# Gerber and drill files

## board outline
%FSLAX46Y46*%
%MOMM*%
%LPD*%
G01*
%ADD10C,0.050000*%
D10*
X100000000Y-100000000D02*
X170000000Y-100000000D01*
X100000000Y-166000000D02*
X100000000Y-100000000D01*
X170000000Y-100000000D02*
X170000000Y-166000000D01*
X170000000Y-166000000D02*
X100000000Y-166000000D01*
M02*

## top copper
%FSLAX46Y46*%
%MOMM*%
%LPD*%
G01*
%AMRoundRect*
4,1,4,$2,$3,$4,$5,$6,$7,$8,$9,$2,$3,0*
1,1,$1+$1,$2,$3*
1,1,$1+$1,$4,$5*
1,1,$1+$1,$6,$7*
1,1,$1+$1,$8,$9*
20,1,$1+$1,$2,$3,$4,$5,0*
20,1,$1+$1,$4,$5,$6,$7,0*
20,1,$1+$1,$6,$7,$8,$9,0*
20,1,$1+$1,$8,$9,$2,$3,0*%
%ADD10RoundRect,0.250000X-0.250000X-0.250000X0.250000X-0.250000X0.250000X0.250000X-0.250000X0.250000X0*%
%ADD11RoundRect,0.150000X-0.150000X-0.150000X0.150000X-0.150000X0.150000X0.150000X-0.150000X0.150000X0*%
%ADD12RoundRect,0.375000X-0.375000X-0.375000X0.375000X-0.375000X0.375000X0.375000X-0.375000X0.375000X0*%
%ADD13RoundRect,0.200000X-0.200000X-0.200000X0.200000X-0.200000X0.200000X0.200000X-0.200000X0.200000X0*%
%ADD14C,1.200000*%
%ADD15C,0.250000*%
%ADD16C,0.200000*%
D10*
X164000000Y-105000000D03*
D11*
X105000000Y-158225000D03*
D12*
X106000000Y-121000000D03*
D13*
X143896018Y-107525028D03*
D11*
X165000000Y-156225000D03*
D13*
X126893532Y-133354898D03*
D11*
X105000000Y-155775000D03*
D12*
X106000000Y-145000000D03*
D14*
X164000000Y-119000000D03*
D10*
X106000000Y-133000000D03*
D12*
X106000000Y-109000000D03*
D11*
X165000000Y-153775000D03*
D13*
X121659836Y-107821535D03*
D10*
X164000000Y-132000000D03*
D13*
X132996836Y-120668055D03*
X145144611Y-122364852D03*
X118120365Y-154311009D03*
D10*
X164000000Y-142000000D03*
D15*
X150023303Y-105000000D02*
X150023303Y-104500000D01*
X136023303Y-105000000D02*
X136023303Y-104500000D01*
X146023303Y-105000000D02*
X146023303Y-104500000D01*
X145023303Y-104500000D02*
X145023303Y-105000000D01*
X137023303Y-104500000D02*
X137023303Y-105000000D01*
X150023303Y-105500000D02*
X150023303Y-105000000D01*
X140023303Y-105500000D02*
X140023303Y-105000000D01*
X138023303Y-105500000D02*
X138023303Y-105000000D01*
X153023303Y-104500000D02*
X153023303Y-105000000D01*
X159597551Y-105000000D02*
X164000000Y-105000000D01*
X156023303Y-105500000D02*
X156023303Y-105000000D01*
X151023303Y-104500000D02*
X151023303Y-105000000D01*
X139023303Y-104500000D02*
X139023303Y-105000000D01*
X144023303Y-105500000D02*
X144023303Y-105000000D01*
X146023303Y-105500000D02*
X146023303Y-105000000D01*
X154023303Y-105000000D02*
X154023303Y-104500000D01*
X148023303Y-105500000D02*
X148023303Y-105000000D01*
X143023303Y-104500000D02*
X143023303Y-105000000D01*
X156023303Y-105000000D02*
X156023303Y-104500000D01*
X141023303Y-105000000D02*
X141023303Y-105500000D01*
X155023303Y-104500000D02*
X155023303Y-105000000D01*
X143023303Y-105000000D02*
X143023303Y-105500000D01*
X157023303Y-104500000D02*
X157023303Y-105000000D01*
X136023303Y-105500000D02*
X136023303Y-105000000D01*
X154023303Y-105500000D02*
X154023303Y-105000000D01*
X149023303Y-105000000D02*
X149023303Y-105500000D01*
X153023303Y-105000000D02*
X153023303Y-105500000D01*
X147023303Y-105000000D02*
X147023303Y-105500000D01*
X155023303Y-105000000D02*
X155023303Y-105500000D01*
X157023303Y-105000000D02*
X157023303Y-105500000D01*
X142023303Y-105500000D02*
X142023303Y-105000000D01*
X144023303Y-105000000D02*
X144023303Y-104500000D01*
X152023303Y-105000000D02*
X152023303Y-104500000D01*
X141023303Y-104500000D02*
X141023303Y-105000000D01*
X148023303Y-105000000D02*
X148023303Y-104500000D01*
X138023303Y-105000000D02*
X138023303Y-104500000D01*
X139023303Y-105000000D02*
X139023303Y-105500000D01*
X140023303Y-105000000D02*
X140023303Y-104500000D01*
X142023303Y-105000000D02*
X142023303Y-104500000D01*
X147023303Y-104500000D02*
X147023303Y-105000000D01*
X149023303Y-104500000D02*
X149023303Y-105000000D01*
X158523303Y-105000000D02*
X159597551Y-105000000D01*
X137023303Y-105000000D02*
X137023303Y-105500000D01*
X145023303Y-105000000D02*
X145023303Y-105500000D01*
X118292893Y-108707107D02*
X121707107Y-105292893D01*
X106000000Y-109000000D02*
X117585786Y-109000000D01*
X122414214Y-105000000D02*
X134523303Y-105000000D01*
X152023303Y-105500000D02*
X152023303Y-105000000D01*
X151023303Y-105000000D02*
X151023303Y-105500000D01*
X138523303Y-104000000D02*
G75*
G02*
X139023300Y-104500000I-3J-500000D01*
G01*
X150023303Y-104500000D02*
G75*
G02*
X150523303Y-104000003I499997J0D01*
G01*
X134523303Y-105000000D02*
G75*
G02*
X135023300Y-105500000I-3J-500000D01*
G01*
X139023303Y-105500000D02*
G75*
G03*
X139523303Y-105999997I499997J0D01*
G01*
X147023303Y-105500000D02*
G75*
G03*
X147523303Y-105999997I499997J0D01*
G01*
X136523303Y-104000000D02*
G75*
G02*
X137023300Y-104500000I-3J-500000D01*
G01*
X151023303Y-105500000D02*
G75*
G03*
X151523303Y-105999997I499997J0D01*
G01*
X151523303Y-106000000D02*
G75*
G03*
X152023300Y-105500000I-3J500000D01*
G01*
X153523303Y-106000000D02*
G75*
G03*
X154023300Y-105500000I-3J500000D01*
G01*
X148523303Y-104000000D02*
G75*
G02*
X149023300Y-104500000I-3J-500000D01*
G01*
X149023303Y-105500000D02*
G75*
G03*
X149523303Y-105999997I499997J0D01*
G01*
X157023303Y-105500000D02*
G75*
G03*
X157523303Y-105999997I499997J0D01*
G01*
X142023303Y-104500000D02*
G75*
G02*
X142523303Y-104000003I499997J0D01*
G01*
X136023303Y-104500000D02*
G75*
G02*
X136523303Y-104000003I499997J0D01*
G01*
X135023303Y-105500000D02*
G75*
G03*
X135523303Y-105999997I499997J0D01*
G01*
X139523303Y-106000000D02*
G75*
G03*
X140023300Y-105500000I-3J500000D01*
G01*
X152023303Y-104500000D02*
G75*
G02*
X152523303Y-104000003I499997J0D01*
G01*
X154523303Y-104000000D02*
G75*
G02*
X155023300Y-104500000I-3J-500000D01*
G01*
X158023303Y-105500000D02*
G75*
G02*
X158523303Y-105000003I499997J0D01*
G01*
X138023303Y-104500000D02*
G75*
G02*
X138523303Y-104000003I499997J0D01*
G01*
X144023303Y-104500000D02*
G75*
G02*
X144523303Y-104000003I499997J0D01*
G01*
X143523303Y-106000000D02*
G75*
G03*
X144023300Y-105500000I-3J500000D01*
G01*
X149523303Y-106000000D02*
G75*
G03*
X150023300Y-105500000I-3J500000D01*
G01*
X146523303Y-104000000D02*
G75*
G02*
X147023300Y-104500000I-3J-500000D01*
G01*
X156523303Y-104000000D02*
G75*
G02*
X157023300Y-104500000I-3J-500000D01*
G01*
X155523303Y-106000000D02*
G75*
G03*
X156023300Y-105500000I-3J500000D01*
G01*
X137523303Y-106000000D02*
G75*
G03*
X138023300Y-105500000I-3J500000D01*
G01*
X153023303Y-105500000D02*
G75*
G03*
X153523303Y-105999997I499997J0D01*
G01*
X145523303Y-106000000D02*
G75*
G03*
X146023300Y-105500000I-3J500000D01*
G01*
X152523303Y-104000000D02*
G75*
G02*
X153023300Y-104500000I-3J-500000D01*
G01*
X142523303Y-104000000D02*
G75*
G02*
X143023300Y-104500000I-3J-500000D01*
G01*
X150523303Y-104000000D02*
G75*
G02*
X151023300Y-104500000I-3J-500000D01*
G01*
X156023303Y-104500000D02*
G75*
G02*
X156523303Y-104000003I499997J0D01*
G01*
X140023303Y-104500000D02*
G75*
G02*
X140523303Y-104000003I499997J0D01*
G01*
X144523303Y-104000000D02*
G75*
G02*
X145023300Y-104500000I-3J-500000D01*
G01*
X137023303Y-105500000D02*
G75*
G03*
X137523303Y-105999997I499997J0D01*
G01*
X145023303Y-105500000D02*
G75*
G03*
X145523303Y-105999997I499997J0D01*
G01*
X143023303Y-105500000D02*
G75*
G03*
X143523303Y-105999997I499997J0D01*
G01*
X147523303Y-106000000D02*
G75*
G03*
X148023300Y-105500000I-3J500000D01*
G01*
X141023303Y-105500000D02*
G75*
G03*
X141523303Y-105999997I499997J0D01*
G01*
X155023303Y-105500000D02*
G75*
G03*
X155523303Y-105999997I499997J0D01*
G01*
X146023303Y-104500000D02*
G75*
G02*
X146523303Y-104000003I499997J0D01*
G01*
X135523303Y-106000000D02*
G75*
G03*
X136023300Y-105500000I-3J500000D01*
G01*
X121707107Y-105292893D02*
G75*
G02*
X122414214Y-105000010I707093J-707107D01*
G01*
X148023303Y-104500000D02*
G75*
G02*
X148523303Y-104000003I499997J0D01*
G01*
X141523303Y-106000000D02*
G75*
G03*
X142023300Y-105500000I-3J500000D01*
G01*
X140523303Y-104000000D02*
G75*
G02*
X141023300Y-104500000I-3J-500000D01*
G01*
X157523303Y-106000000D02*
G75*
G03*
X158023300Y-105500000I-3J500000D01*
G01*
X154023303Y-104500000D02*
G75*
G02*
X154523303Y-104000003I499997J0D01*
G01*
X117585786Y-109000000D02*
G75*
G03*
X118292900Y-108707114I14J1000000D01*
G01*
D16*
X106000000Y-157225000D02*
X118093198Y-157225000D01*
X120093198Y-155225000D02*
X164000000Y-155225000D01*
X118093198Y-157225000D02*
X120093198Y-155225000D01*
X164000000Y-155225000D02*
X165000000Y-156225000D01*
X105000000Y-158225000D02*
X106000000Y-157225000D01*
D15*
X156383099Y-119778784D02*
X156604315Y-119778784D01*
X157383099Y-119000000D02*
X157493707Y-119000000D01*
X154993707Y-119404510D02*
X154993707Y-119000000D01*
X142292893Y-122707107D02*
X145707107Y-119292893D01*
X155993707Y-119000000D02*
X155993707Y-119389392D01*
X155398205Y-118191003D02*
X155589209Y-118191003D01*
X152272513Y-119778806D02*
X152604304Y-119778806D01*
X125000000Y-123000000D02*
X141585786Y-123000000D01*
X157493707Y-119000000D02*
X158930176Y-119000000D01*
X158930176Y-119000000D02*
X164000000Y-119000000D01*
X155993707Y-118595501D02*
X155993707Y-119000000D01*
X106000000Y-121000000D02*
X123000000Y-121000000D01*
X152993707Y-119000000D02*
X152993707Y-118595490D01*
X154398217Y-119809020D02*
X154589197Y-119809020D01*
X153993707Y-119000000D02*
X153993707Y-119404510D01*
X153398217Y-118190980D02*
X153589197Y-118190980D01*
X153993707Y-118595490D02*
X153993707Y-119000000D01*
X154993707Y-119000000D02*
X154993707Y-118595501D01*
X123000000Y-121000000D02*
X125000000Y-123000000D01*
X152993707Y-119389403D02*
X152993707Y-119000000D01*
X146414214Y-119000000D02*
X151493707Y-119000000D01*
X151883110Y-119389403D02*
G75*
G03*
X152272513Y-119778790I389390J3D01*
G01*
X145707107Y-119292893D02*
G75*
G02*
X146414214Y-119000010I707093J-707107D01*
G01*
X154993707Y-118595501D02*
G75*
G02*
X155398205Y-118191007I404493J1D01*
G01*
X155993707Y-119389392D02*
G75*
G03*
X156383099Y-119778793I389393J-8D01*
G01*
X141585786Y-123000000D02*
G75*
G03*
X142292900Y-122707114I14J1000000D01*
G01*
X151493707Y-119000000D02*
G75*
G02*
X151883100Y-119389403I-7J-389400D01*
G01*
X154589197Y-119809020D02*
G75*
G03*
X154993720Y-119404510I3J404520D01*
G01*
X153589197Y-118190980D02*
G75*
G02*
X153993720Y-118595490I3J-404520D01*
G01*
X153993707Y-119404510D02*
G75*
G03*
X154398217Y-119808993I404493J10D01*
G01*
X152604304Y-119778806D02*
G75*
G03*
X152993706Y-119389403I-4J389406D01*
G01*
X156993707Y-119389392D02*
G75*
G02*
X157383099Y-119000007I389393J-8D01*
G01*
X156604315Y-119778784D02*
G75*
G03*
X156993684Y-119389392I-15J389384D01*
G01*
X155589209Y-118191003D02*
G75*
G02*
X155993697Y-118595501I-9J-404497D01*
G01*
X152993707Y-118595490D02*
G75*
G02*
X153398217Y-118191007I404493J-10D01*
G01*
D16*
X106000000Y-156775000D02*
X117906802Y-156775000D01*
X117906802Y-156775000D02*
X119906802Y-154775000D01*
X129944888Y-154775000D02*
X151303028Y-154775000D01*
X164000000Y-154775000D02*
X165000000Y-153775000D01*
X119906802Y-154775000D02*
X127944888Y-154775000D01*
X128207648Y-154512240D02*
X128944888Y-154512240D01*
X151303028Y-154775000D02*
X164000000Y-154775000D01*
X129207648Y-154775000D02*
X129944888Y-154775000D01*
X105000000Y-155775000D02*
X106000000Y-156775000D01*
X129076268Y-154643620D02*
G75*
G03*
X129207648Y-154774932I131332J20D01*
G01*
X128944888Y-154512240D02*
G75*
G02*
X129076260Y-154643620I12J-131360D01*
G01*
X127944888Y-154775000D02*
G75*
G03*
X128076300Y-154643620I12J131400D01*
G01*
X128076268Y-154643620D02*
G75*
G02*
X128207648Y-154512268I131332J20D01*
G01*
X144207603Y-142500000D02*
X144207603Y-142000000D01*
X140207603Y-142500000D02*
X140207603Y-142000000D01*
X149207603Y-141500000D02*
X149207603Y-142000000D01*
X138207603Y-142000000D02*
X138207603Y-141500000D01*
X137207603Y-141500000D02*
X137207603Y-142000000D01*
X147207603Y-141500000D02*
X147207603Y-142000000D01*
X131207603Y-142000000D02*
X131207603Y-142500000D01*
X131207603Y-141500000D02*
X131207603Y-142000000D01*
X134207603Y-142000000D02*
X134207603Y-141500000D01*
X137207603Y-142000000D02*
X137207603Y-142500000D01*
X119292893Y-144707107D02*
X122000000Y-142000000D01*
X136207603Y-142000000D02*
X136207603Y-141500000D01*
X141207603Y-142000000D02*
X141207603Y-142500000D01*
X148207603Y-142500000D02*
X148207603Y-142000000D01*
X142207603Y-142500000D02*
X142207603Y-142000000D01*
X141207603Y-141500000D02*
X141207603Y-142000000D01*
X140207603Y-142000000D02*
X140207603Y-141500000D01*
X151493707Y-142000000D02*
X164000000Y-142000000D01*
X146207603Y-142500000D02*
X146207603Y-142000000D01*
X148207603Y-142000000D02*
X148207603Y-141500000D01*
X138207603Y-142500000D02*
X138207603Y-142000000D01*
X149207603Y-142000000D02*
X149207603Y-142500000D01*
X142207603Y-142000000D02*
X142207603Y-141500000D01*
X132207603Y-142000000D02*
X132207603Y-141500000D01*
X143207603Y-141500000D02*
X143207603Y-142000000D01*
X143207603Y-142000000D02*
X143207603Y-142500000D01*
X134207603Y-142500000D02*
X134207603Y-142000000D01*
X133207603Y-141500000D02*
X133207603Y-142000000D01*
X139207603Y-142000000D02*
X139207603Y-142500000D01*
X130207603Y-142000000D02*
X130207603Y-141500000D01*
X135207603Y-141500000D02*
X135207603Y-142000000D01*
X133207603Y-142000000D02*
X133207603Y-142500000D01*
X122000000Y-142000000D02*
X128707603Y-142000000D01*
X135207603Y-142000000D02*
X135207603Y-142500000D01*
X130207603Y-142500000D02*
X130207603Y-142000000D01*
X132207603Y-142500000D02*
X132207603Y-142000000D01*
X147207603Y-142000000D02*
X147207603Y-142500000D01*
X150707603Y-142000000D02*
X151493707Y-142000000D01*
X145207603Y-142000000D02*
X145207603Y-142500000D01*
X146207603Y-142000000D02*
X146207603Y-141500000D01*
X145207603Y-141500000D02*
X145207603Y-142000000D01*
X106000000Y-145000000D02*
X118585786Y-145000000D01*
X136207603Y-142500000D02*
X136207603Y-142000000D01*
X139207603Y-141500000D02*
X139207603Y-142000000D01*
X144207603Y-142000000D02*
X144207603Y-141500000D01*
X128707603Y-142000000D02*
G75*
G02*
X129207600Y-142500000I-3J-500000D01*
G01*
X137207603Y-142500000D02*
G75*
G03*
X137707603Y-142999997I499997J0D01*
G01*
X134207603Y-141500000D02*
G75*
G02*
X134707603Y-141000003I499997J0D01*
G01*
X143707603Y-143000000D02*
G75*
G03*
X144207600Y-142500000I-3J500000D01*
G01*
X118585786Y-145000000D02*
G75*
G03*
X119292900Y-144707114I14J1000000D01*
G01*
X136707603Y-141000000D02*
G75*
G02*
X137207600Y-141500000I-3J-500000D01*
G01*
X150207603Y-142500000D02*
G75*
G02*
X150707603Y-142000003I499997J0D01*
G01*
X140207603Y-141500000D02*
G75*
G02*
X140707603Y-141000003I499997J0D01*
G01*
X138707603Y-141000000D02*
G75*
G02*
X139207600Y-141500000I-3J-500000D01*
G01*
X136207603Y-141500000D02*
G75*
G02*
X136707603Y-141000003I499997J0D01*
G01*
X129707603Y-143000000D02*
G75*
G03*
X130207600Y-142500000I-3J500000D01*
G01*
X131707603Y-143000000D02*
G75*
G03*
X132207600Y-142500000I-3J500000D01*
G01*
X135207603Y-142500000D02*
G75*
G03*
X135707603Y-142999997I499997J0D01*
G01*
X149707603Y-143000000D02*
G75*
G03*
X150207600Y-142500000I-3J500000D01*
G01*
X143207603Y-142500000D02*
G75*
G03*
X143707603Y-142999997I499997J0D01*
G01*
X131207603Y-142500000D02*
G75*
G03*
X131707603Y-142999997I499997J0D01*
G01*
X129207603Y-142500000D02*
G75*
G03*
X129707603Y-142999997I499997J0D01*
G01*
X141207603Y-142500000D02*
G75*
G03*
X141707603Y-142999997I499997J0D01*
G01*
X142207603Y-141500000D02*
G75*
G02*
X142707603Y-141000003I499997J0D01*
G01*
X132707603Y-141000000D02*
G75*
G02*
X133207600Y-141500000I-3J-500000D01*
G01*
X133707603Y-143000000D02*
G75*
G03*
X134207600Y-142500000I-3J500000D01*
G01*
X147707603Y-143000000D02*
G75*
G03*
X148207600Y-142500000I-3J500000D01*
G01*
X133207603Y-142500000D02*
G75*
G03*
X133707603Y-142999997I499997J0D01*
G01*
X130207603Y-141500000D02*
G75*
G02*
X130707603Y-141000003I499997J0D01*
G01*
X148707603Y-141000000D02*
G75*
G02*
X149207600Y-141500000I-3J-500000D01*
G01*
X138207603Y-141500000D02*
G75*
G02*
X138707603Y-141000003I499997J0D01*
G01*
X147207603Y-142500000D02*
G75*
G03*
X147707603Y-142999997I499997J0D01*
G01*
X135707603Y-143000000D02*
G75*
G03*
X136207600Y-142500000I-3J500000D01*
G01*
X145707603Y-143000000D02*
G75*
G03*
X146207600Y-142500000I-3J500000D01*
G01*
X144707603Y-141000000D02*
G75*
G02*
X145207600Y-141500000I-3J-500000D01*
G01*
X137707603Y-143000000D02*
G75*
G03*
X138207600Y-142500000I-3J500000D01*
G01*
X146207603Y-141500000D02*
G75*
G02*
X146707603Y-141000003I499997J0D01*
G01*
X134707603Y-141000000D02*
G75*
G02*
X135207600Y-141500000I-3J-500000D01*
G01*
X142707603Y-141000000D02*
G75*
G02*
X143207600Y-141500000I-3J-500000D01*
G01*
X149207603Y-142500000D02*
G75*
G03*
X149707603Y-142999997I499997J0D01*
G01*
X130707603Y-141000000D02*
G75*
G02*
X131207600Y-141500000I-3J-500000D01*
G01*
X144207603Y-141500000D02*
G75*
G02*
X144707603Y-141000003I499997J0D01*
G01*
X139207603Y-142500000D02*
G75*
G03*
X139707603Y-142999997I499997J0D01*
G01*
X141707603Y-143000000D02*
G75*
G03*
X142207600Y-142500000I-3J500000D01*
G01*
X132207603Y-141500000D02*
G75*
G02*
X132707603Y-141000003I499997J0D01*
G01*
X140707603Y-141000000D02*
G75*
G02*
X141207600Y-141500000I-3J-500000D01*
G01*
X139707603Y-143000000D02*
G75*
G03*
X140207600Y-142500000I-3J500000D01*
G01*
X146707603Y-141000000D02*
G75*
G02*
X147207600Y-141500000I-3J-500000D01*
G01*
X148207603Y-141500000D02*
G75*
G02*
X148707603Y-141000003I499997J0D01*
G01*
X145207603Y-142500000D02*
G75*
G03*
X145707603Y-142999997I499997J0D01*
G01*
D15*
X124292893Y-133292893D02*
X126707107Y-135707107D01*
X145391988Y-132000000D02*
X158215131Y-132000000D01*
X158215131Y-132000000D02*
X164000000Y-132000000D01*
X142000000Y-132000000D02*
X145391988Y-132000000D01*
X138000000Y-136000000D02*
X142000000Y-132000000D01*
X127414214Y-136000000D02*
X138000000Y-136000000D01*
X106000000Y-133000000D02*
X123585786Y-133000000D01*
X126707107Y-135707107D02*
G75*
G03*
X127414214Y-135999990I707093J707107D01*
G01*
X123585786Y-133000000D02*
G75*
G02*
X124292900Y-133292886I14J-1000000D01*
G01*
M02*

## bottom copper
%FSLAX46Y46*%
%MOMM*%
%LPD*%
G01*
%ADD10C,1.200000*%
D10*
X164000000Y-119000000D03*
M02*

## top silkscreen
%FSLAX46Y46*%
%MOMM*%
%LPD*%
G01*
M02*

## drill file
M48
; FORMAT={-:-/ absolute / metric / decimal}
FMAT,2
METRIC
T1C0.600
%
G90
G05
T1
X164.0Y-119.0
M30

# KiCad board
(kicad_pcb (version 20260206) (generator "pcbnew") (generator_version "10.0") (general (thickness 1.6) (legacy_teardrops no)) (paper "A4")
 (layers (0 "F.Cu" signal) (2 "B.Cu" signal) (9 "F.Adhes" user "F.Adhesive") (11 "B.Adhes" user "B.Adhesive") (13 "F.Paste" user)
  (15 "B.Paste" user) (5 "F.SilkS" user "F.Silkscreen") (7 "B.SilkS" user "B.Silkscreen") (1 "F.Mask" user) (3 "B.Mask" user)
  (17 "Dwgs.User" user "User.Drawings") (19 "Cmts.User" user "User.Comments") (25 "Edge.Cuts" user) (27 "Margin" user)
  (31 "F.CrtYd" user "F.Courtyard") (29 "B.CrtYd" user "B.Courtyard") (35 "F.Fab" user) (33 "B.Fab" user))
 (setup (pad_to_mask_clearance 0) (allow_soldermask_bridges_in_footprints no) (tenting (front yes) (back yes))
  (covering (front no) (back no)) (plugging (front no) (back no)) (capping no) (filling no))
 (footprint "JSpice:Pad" (layer "F.Cu") (at 164 105)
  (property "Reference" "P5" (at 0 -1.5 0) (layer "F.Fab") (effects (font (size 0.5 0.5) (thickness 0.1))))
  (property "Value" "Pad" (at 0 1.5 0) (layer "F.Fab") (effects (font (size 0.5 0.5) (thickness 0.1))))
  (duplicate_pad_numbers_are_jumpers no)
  (pad "1" smd roundrect (at 0 0) (size 1 1) (layers "F.Cu" "F.Mask") (roundrect_rratio 0.25) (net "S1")))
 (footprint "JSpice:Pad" (layer "F.Cu") (at 105 158.225)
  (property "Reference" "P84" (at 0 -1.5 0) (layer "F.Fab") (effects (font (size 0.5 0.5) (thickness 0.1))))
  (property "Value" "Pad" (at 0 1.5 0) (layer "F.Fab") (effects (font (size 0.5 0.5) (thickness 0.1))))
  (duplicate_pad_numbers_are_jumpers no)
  (pad "1" smd roundrect (at 0 0) (size 0.6 0.6) (layers "F.Cu" "F.Mask") (roundrect_rratio 0.25) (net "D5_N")))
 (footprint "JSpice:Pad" (layer "F.Cu") (at 106 121)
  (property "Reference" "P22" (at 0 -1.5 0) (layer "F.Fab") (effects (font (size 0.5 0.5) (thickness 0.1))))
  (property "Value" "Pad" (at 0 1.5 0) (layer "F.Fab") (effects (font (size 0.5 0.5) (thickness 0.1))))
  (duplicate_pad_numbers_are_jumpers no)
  (pad "1" smd roundrect (at 0 0) (size 1.5 1.5) (layers "F.Cu" "F.Mask") (roundrect_rratio 0.25) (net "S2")))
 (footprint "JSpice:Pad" (layer "F.Cu") (at 143.896018 107.525028)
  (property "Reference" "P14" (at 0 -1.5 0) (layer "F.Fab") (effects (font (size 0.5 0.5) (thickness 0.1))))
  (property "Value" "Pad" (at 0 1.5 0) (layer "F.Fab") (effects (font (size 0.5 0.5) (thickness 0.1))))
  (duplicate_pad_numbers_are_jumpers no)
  (pad "1" smd roundrect (at 0 0) (size 0.8 0.8) (layers "F.Cu" "F.Mask") (roundrect_rratio 0.25) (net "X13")))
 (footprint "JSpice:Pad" (layer "F.Cu") (at 165 156.225)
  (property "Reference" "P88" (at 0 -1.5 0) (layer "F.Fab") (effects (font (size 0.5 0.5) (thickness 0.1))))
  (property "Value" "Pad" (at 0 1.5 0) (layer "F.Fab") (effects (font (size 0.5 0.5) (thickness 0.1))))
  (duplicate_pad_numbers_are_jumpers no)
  (pad "1" smd roundrect (at 0 0) (size 0.6 0.6) (layers "F.Cu" "F.Mask") (roundrect_rratio 0.25) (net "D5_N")))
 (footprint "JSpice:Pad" (layer "F.Cu") (at 126.893532 133.354898)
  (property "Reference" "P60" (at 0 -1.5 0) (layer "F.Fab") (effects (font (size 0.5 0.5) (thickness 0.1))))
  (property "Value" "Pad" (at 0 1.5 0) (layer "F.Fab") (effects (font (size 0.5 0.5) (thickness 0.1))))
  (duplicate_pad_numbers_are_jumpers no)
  (pad "1" smd roundrect (at 0 0) (size 0.8 0.8) (layers "F.Cu" "F.Mask") (roundrect_rratio 0.25) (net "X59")))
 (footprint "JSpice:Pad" (layer "F.Cu") (at 105 155.775)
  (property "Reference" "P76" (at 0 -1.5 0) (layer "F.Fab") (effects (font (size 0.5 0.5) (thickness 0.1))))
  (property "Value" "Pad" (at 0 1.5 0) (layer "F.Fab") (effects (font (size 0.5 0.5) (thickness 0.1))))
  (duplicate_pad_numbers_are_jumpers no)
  (pad "1" smd roundrect (at 0 0) (size 0.6 0.6) (layers "F.Cu" "F.Mask") (roundrect_rratio 0.25) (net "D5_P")))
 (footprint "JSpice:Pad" (layer "F.Cu") (at 106 145)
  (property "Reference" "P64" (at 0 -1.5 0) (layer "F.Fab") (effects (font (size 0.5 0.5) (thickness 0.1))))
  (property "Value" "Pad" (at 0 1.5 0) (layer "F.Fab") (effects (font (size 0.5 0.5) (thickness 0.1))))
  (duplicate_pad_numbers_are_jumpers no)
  (pad "1" smd roundrect (at 0 0) (size 1.5 1.5) (layers "F.Cu" "F.Mask") (roundrect_rratio 0.25) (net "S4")))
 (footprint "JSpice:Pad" (layer "F.Cu") (at 164 119)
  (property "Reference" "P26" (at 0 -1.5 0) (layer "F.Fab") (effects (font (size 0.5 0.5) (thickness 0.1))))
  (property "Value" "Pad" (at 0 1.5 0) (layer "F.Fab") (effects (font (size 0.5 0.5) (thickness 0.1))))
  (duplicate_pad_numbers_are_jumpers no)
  (pad "1" thru_hole circle (at 0 0) (size 1.2 1.2) (drill 0.6) (layers "*.Cu" "*.Mask") (remove_unused_layers no) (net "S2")))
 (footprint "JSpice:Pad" (layer "F.Cu") (at 106 133)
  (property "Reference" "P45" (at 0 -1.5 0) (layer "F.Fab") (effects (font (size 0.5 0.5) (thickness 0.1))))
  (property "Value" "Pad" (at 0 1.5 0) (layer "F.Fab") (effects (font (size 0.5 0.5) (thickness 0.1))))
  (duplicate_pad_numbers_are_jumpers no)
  (pad "1" smd roundrect (at 0 0) (size 1 1) (layers "F.Cu" "F.Mask") (roundrect_rratio 0.25) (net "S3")))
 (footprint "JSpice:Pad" (layer "F.Cu") (at 106 109)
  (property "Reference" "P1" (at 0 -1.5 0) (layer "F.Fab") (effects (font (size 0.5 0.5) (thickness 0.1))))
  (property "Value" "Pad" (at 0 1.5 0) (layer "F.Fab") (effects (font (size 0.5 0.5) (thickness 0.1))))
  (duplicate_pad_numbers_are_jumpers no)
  (pad "1" smd roundrect (at 0 0) (size 1.5 1.5) (layers "F.Cu" "F.Mask") (roundrect_rratio 0.25) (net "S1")))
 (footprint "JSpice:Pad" (layer "F.Cu") (at 165 153.775)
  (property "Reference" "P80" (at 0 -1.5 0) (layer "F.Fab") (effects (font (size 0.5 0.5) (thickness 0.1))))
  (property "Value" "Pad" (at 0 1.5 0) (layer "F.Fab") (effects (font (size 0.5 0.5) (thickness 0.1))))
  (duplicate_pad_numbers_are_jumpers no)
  (pad "1" smd roundrect (at 0 0) (size 0.6 0.6) (layers "F.Cu" "F.Mask") (roundrect_rratio 0.25) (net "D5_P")))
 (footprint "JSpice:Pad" (layer "F.Cu") (at 121.659836 107.821535)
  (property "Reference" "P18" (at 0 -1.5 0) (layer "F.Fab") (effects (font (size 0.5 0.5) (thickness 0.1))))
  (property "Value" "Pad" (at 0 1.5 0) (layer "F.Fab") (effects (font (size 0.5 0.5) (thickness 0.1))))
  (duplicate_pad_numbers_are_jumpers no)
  (pad "1" smd roundrect (at 0 0) (size 0.8 0.8) (layers "F.Cu" "F.Mask") (roundrect_rratio 0.25) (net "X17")))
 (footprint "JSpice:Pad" (layer "F.Cu") (at 164 132)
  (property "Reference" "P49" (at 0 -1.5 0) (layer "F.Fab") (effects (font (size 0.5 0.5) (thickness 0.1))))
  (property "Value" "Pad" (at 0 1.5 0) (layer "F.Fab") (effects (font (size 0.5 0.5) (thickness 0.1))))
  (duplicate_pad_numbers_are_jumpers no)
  (pad "1" smd roundrect (at 0 0) (size 1 1) (layers "F.Cu" "F.Mask") (roundrect_rratio 0.25) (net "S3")))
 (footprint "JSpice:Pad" (layer "F.Cu") (at 132.996836 120.668055)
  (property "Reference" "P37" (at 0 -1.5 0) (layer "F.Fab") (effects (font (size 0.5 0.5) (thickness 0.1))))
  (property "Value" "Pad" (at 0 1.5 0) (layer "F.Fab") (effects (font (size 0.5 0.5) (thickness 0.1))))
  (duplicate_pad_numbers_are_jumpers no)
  (pad "1" smd roundrect (at 0 0) (size 0.8 0.8) (layers "F.Cu" "F.Mask") (roundrect_rratio 0.25) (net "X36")))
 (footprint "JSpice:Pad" (layer "F.Cu") (at 145.144611 122.364852)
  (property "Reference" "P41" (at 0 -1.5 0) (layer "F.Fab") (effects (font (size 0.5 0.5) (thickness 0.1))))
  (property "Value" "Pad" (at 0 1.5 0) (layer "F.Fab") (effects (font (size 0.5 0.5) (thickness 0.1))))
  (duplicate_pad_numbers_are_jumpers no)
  (pad "1" smd roundrect (at 0 0) (size 0.8 0.8) (layers "F.Cu" "F.Mask") (roundrect_rratio 0.25) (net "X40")))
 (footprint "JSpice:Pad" (layer "F.Cu") (at 118.120365 154.311009)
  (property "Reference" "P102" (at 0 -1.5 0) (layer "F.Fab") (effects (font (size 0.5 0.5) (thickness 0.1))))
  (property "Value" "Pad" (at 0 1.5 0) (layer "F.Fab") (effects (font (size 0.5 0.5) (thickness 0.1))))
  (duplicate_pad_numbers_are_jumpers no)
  (pad "1" smd roundrect (at 0 0) (size 0.8 0.8) (layers "F.Cu" "F.Mask") (roundrect_rratio 0.25) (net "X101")))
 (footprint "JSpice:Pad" (layer "F.Cu") (at 164 142)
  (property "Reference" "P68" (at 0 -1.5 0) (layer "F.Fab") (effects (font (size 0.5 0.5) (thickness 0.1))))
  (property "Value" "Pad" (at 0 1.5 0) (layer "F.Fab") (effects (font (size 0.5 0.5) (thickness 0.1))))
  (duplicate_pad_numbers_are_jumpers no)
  (pad "1" smd roundrect (at 0 0) (size 1 1) (layers "F.Cu" "F.Mask") (roundrect_rratio 0.25) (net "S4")))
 (gr_line (start 100 100) (end 170 100) (stroke (width 0.05) (type default)) (layer "Edge.Cuts"))
 (gr_line (start 100 166) (end 100 100) (stroke (width 0.05) (type default)) (layer "Edge.Cuts"))
 (gr_line (start 170 100) (end 170 166) (stroke (width 0.05) (type default)) (layer "Edge.Cuts"))
 (gr_line (start 170 166) (end 100 166) (stroke (width 0.05) (type default)) (layer "Edge.Cuts"))
 (segment (start 150.023303 105) (end 150.023303 104.5) (width 0.25) (layer "F.Cu") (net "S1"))
 (segment (start 136.023303 105) (end 136.023303 104.5) (width 0.25) (layer "F.Cu") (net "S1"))
 (segment (start 146.023303 105) (end 146.023303 104.5) (width 0.25) (layer "F.Cu") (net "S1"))
 (segment (start 145.023303 104.5) (end 145.023303 105) (width 0.25) (layer "F.Cu") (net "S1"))
 (segment (start 137.023303 104.5) (end 137.023303 105) (width 0.25) (layer "F.Cu") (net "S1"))
 (segment (start 150.023303 105.5) (end 150.023303 105) (width 0.25) (layer "F.Cu") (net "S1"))
 (segment (start 140.023303 105.5) (end 140.023303 105) (width 0.25) (layer "F.Cu") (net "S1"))
 (segment (start 138.023303 105.5) (end 138.023303 105) (width 0.25) (layer "F.Cu") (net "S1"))
 (segment (start 153.023303 104.5) (end 153.023303 105) (width 0.25) (layer "F.Cu") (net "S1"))
 (segment (start 159.597551 105) (end 164 105) (width 0.25) (layer "F.Cu") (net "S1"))
 (segment (start 156.023303 105.5) (end 156.023303 105) (width 0.25) (layer "F.Cu") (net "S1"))
 (segment (start 151.023303 104.5) (end 151.023303 105) (width 0.25) (layer "F.Cu") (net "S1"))
 (segment (start 139.023303 104.5) (end 139.023303 105) (width 0.25) (layer "F.Cu") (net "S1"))
 (segment (start 144.023303 105.5) (end 144.023303 105) (width 0.25) (layer "F.Cu") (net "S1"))
 (segment (start 146.023303 105.5) (end 146.023303 105) (width 0.25) (layer "F.Cu") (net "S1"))
 (segment (start 154.023303 105) (end 154.023303 104.5) (width 0.25) (layer "F.Cu") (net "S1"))
 (segment (start 148.023303 105.5) (end 148.023303 105) (width 0.25) (layer "F.Cu") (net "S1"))
 (segment (start 143.023303 104.5) (end 143.023303 105) (width 0.25) (layer "F.Cu") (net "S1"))
 (segment (start 156.023303 105) (end 156.023303 104.5) (width 0.25) (layer "F.Cu") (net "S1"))
 (segment (start 141.023303 105) (end 141.023303 105.5) (width 0.25) (layer "F.Cu") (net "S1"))
 (segment (start 155.023303 104.5) (end 155.023303 105) (width 0.25) (layer "F.Cu") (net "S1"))
 (segment (start 143.023303 105) (end 143.023303 105.5) (width 0.25) (layer "F.Cu") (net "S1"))
 (segment (start 157.023303 104.5) (end 157.023303 105) (width 0.25) (layer "F.Cu") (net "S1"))
 (segment (start 136.023303 105.5) (end 136.023303 105) (width 0.25) (layer "F.Cu") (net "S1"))
 (segment (start 154.023303 105.5) (end 154.023303 105) (width 0.25) (layer "F.Cu") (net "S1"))
 (segment (start 149.023303 105) (end 149.023303 105.5) (width 0.25) (layer "F.Cu") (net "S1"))
 (segment (start 153.023303 105) (end 153.023303 105.5) (width 0.25) (layer "F.Cu") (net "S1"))
 (segment (start 147.023303 105) (end 147.023303 105.5) (width 0.25) (layer "F.Cu") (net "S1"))
 (segment (start 155.023303 105) (end 155.023303 105.5) (width 0.25) (layer "F.Cu") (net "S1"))
 (segment (start 157.023303 105) (end 157.023303 105.5) (width 0.25) (layer "F.Cu") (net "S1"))
 (segment (start 142.023303 105.5) (end 142.023303 105) (width 0.25) (layer "F.Cu") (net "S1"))
 (segment (start 144.023303 105) (end 144.023303 104.5) (width 0.25) (layer "F.Cu") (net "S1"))
 (segment (start 152.023303 105) (end 152.023303 104.5) (width 0.25) (layer "F.Cu") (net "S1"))
 (segment (start 141.023303 104.5) (end 141.023303 105) (width 0.25) (layer "F.Cu") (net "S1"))
 (segment (start 148.023303 105) (end 148.023303 104.5) (width 0.25) (layer "F.Cu") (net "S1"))
 (segment (start 138.023303 105) (end 138.023303 104.5) (width 0.25) (layer "F.Cu") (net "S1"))
 (segment (start 139.023303 105) (end 139.023303 105.5) (width 0.25) (layer "F.Cu") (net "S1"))
 (segment (start 140.023303 105) (end 140.023303 104.5) (width 0.25) (layer "F.Cu") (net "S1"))
 (segment (start 142.023303 105) (end 142.023303 104.5) (width 0.25) (layer "F.Cu") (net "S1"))
 (segment (start 147.023303 104.5) (end 147.023303 105) (width 0.25) (layer "F.Cu") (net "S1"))
 (segment (start 149.023303 104.5) (end 149.023303 105) (width 0.25) (layer "F.Cu") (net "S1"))
 (segment (start 158.523303 105) (end 159.597551 105) (width 0.25) (layer "F.Cu") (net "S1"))
 (segment (start 137.023303 105) (end 137.023303 105.5) (width 0.25) (layer "F.Cu") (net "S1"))
 (segment (start 145.023303 105) (end 145.023303 105.5) (width 0.25) (layer "F.Cu") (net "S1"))
 (segment (start 118.292893 108.707107) (end 121.707107 105.292893) (width 0.25) (layer "F.Cu") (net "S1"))
 (segment (start 106 109) (end 117.585786 109) (width 0.25) (layer "F.Cu") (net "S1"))
 (segment (start 122.414214 105) (end 134.523303 105) (width 0.25) (layer "F.Cu") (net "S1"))
 (segment (start 152.023303 105.5) (end 152.023303 105) (width 0.25) (layer "F.Cu") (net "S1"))
 (segment (start 151.023303 105) (end 151.023303 105.5) (width 0.25) (layer "F.Cu") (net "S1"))
 (arc (start 138.523303 104) (mid 138.876856 104.146447) (end 139.023303 104.5) (width 0.25) (layer "F.Cu") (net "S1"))
 (arc (start 150.023303 104.5) (mid 150.16975 104.146447) (end 150.523303 104) (width 0.25) (layer "F.Cu") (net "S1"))
 (arc (start 134.523303 105) (mid 134.876856 105.146447) (end 135.023303 105.5) (width 0.25) (layer "F.Cu") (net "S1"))
 (arc (start 139.023303 105.5) (mid 139.16975 105.853553) (end 139.523303 106) (width 0.25) (layer "F.Cu") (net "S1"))
 (arc (start 147.023303 105.5) (mid 147.16975 105.853553) (end 147.523303 106) (width 0.25) (layer "F.Cu") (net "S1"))
 (arc (start 136.523303 104) (mid 136.876856 104.146447) (end 137.023303 104.5) (width 0.25) (layer "F.Cu") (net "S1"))
 (arc (start 151.023303 105.5) (mid 151.16975 105.853553) (end 151.523303 106) (width 0.25) (layer "F.Cu") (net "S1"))
 (arc (start 151.523303 106) (mid 151.876856 105.853553) (end 152.023303 105.5) (width 0.25) (layer "F.Cu") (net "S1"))
 (arc (start 153.523303 106) (mid 153.876856 105.853553) (end 154.023303 105.5) (width 0.25) (layer "F.Cu") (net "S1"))
 (arc (start 148.523303 104) (mid 148.876856 104.146447) (end 149.023303 104.5) (width 0.25) (layer "F.Cu") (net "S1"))
 (arc (start 149.023303 105.5) (mid 149.16975 105.853553) (end 149.523303 106) (width 0.25) (layer "F.Cu") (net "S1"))
 (arc (start 157.023303 105.5) (mid 157.16975 105.853553) (end 157.523303 106) (width 0.25) (layer "F.Cu") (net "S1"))
 (arc (start 142.023303 104.5) (mid 142.16975 104.146447) (end 142.523303 104) (width 0.25) (layer "F.Cu") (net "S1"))
 (arc (start 136.023303 104.5) (mid 136.16975 104.146447) (end 136.523303 104) (width 0.25) (layer "F.Cu") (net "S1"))
 (arc (start 135.023303 105.5) (mid 135.16975 105.853553) (end 135.523303 106) (width 0.25) (layer "F.Cu") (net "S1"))
 (arc (start 139.523303 106) (mid 139.876856 105.853553) (end 140.023303 105.5) (width 0.25) (layer "F.Cu") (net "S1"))
 (arc (start 152.023303 104.5) (mid 152.16975 104.146447) (end 152.523303 104) (width 0.25) (layer "F.Cu") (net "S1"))
 (arc (start 154.523303 104) (mid 154.876856 104.146447) (end 155.023303 104.5) (width 0.25) (layer "F.Cu") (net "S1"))
 (arc (start 158.023303 105.5) (mid 158.16975 105.146447) (end 158.523303 105) (width 0.25) (layer "F.Cu") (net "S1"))
 (arc (start 138.023303 104.5) (mid 138.16975 104.146447) (end 138.523303 104) (width 0.25) (layer "F.Cu") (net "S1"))
 (arc (start 144.023303 104.5) (mid 144.16975 104.146447) (end 144.523303 104) (width 0.25) (layer "F.Cu") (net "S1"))
 (arc (start 143.523303 106) (mid 143.876856 105.853553) (end 144.023303 105.5) (width 0.25) (layer "F.Cu") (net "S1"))
 (arc (start 149.523303 106) (mid 149.876856 105.853553) (end 150.023303 105.5) (width 0.25) (layer "F.Cu") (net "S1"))
 (arc (start 146.523303 104) (mid 146.876856 104.146447) (end 147.023303 104.5) (width 0.25) (layer "F.Cu") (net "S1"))
 (arc (start 156.523303 104) (mid 156.876856 104.146447) (end 157.023303 104.5) (width 0.25) (layer "F.Cu") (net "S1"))
 (arc (start 155.523303 106) (mid 155.876856 105.853553) (end 156.023303 105.5) (width 0.25) (layer "F.Cu") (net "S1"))
 (arc (start 137.523303 106) (mid 137.876856 105.853553) (end 138.023303 105.5) (width 0.25) (layer "F.Cu") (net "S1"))
 (arc (start 153.023303 105.5) (mid 153.16975 105.853553) (end 153.523303 106) (width 0.25) (layer "F.Cu") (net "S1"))
 (arc (start 145.523303 106) (mid 145.876856 105.853553) (end 146.023303 105.5) (width 0.25) (layer "F.Cu") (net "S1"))
 (arc (start 152.523303 104) (mid 152.876856 104.146447) (end 153.023303 104.5) (width 0.25) (layer "F.Cu") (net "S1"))
 (arc (start 142.523303 104) (mid 142.876856 104.146447) (end 143.023303 104.5) (width 0.25) (layer "F.Cu") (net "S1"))
 (arc (start 150.523303 104) (mid 150.876856 104.146447) (end 151.023303 104.5) (width 0.25) (layer "F.Cu") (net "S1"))
 (arc (start 156.023303 104.5) (mid 156.16975 104.146447) (end 156.523303 104) (width 0.25) (layer "F.Cu") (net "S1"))
 (arc (start 140.023303 104.5) (mid 140.16975 104.146447) (end 140.523303 104) (width 0.25) (layer "F.Cu") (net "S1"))
 (arc (start 144.523303 104) (mid 144.876856 104.146447) (end 145.023303 104.5) (width 0.25) (layer "F.Cu") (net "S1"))
 (arc (start 137.023303 105.5) (mid 137.16975 105.853553) (end 137.523303 106) (width 0.25) (layer "F.Cu") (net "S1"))
 (arc (start 145.023303 105.5) (mid 145.16975 105.853553) (end 145.523303 106) (width 0.25) (layer "F.Cu") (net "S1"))
 (arc (start 143.023303 105.5) (mid 143.16975 105.853553) (end 143.523303 106) (width 0.25) (layer "F.Cu") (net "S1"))
 (arc (start 147.523303 106) (mid 147.876856 105.853553) (end 148.023303 105.5) (width 0.25) (layer "F.Cu") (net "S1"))
 (arc (start 141.023303 105.5) (mid 141.16975 105.853553) (end 141.523303 106) (width 0.25) (layer "F.Cu") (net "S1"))
 (arc (start 155.023303 105.5) (mid 155.16975 105.853553) (end 155.523303 106) (width 0.25) (layer "F.Cu") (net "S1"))
 (arc (start 146.023303 104.5) (mid 146.16975 104.146447) (end 146.523303 104) (width 0.25) (layer "F.Cu") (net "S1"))
 (arc (start 135.523303 106) (mid 135.876856 105.853553) (end 136.023303 105.5) (width 0.25) (layer "F.Cu") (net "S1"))
 (arc (start 121.707107 105.292893) (mid 122.03153 105.07612) (end 122.414214 105) (width 0.25) (layer "F.Cu") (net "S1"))
 (arc (start 148.023303 104.5) (mid 148.16975 104.146447) (end 148.523303 104) (width 0.25) (layer "F.Cu") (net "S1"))
 (arc (start 141.523303 106) (mid 141.876856 105.853553) (end 142.023303 105.5) (width 0.25) (layer "F.Cu") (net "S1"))
 (arc (start 140.523303 104) (mid 140.876856 104.146447) (end 141.023303 104.5) (width 0.25) (layer "F.Cu") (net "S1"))
 (arc (start 157.523303 106) (mid 157.876856 105.853553) (end 158.023303 105.5) (width 0.25) (layer "F.Cu") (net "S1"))
 (arc (start 154.023303 104.5) (mid 154.16975 104.146447) (end 154.523303 104) (width 0.25) (layer "F.Cu") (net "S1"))
 (arc (start 117.585786 109) (mid 117.96847 108.92388) (end 118.292893 108.707107) (width 0.25) (layer "F.Cu") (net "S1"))
 (segment (start 106 157.225) (end 118.093198 157.225) (width 0.2) (layer "F.Cu") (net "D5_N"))
 (segment (start 120.093198 155.225) (end 164 155.225) (width 0.2) (layer "F.Cu") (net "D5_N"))
 (segment (start 118.093198 157.225) (end 120.093198 155.225) (width 0.2) (layer "F.Cu") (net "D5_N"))
 (segment (start 164 155.225) (end 165 156.225) (width 0.2) (layer "F.Cu") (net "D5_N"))
 (segment (start 105 158.225) (end 106 157.225) (width 0.2) (layer "F.Cu") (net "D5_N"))
 (segment (start 156.383099 119.778784) (end 156.604315 119.778784) (width 0.25) (layer "F.Cu") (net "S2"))
 (segment (start 157.383099 119) (end 157.493707 119) (width 0.25) (layer "F.Cu") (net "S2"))
 (segment (start 154.993707 119.40451) (end 154.993707 119) (width 0.25) (layer "F.Cu") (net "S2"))
 (segment (start 142.292893 122.707107) (end 145.707107 119.292893) (width 0.25) (layer "F.Cu") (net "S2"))
 (segment (start 155.993707 119) (end 155.993707 119.389392) (width 0.25) (layer "F.Cu") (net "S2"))
 (segment (start 155.398205 118.191003) (end 155.589209 118.191003) (width 0.25) (layer "F.Cu") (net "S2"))
 (segment (start 152.272513 119.778806) (end 152.604304 119.778806) (width 0.25) (layer "F.Cu") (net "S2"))
 (segment (start 125 123) (end 141.585786 123) (width 0.25) (layer "F.Cu") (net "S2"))
 (segment (start 157.493707 119) (end 158.930176 119) (width 0.25) (layer "F.Cu") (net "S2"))
 (segment (start 158.930176 119) (end 164 119) (width 0.25) (layer "F.Cu") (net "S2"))
 (segment (start 155.993707 118.595501) (end 155.993707 119) (width 0.25) (layer "F.Cu") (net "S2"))
 (segment (start 106 121) (end 123 121) (width 0.25) (layer "F.Cu") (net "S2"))
 (segment (start 152.993707 119) (end 152.993707 118.59549) (width 0.25) (layer "F.Cu") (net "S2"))
 (segment (start 154.398217 119.80902) (end 154.589197 119.80902) (width 0.25) (layer "F.Cu") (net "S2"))
 (segment (start 153.993707 119) (end 153.993707 119.40451) (width 0.25) (layer "F.Cu") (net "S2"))
 (segment (start 153.398217 118.19098) (end 153.589197 118.19098) (width 0.25) (layer "F.Cu") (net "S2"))
 (segment (start 153.993707 118.59549) (end 153.993707 119) (width 0.25) (layer "F.Cu") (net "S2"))
 (segment (start 154.993707 119) (end 154.993707 118.595501) (width 0.25) (layer "F.Cu") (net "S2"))
 (segment (start 123 121) (end 125 123) (width 0.25) (layer "F.Cu") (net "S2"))
 (segment (start 152.993707 119.389403) (end 152.993707 119) (width 0.25) (layer "F.Cu") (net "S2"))
 (segment (start 146.414214 119) (end 151.493707 119) (width 0.25) (layer "F.Cu") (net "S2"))
 (arc (start 151.88311 119.389403) (mid 151.997163 119.664753) (end 152.272513 119.778806) (width 0.25) (layer "F.Cu") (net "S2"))
 (arc (start 145.707107 119.292893) (mid 146.03153 119.07612) (end 146.414214 119) (width 0.25) (layer "F.Cu") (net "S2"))
 (arc (start 154.993707 118.595501) (mid 155.112182 118.309478) (end 155.398205 118.191003) (width 0.25) (layer "F.Cu") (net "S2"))
 (arc (start 155.993707 119.389392) (mid 156.107757 119.664734) (end 156.383099 119.778784) (width 0.25) (layer "F.Cu") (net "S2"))
 (arc (start 141.585786 123) (mid 141.96847 122.92388) (end 142.292893 122.707107) (width 0.25) (layer "F.Cu") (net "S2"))
 (arc (start 151.493707 119) (mid 151.769057 119.114053) (end 151.88311 119.389403) (width 0.25) (layer "F.Cu") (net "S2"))
 (arc (start 154.589197 119.80902) (mid 154.875229 119.690542) (end 154.993707 119.40451) (width 0.25) (layer "F.Cu") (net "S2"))
 (arc (start 153.589197 118.19098) (mid 153.875229 118.309458) (end 153.993707 118.59549) (width 0.25) (layer "F.Cu") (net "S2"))
 (arc (start 153.993707 119.40451) (mid 154.112185 119.690542) (end 154.398217 119.80902) (width 0.25) (layer "F.Cu") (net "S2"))
 (arc (start 152.604304 119.778806) (mid 152.879654 119.664753) (end 152.993707 119.389403) (width 0.25) (layer "F.Cu") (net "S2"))
 (arc (start 156.993707 119.389392) (mid 157.107757 119.11405) (end 157.383099 119) (width 0.25) (layer "F.Cu") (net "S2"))
 (arc (start 156.604315 119.778784) (mid 156.879657 119.664734) (end 156.993707 119.389392) (width 0.25) (layer "F.Cu") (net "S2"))
 (arc (start 155.589209 118.191003) (mid 155.875232 118.309478) (end 155.993707 118.595501) (width 0.25) (layer "F.Cu") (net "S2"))
 (arc (start 152.993707 118.59549) (mid 153.112185 118.309458) (end 153.398217 118.19098) (width 0.25) (layer "F.Cu") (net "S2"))
 (segment (start 106 156.775) (end 117.906802 156.775) (width 0.2) (layer "F.Cu") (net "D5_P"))
 (segment (start 117.906802 156.775) (end 119.906802 154.775) (width 0.2) (layer "F.Cu") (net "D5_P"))
 (segment (start 129.944888 154.775) (end 151.303028 154.775) (width 0.2) (layer "F.Cu") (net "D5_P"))
 (segment (start 164 154.775) (end 165 153.775) (width 0.2) (layer "F.Cu") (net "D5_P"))
 (segment (start 119.906802 154.775) (end 127.944888 154.775) (width 0.2) (layer "F.Cu") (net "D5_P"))
 (segment (start 128.207648 154.51224) (end 128.944888 154.51224) (width 0.2) (layer "F.Cu") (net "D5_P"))
 (segment (start 151.303028 154.775) (end 164 154.775) (width 0.2) (layer "F.Cu") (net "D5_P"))
 (segment (start 129.207648 154.775) (end 129.944888 154.775) (width 0.2) (layer "F.Cu") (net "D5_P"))
 (segment (start 105 155.775) (end 106 156.775) (width 0.2) (layer "F.Cu") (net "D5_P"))
 (arc (start 129.076268 154.64362) (mid 129.114748 154.73652) (end 129.207648 154.775) (width 0.2) (layer "F.Cu") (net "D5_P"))
 (arc (start 128.944888 154.51224) (mid 129.037788 154.55072) (end 129.076268 154.64362) (width 0.2) (layer "F.Cu") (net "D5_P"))
 (arc (start 127.944888 154.775) (mid 128.037788 154.73652) (end 128.076268 154.64362) (width 0.2) (layer "F.Cu") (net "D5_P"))
 (arc (start 128.076268 154.64362) (mid 128.114748 154.55072) (end 128.207648 154.51224) (width 0.2) (layer "F.Cu") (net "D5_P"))
 (segment (start 144.207603 142.5) (end 144.207603 142) (width 0.2) (layer "F.Cu") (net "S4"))
 (segment (start 140.207603 142.5) (end 140.207603 142) (width 0.2) (layer "F.Cu") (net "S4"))
 (segment (start 149.207603 141.5) (end 149.207603 142) (width 0.2) (layer "F.Cu") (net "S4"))
 (segment (start 138.207603 142) (end 138.207603 141.5) (width 0.2) (layer "F.Cu") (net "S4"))
 (segment (start 137.207603 141.5) (end 137.207603 142) (width 0.2) (layer "F.Cu") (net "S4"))
 (segment (start 147.207603 141.5) (end 147.207603 142) (width 0.2) (layer "F.Cu") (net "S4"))
 (segment (start 131.207603 142) (end 131.207603 142.5) (width 0.2) (layer "F.Cu") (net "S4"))
 (segment (start 131.207603 141.5) (end 131.207603 142) (width 0.2) (layer "F.Cu") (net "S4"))
 (segment (start 134.207603 142) (end 134.207603 141.5) (width 0.2) (layer "F.Cu") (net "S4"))
 (segment (start 137.207603 142) (end 137.207603 142.5) (width 0.2) (layer "F.Cu") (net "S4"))
 (segment (start 119.292893 144.707107) (end 122 142) (width 0.2) (layer "F.Cu") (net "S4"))
 (segment (start 136.207603 142) (end 136.207603 141.5) (width 0.2) (layer "F.Cu") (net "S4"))
 (segment (start 141.207603 142) (end 141.207603 142.5) (width 0.2) (layer "F.Cu") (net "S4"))
 (segment (start 148.207603 142.5) (end 148.207603 142) (width 0.2) (layer "F.Cu") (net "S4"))
 (segment (start 142.207603 142.5) (end 142.207603 142) (width 0.2) (layer "F.Cu") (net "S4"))
 (segment (start 141.207603 141.5) (end 141.207603 142) (width 0.2) (layer "F.Cu") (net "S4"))
 (segment (start 140.207603 142) (end 140.207603 141.5) (width 0.2) (layer "F.Cu") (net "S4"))
 (segment (start 151.493707 142) (end 164 142) (width 0.2) (layer "F.Cu") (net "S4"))
 (segment (start 146.207603 142.5) (end 146.207603 142) (width 0.2) (layer "F.Cu") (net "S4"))
 (segment (start 148.207603 142) (end 148.207603 141.5) (width 0.2) (layer "F.Cu") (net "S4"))
 (segment (start 138.207603 142.5) (end 138.207603 142) (width 0.2) (layer "F.Cu") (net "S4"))
 (segment (start 149.207603 142) (end 149.207603 142.5) (width 0.2) (layer "F.Cu") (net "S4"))
 (segment (start 142.207603 142) (end 142.207603 141.5) (width 0.2) (layer "F.Cu") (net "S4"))
 (segment (start 132.207603 142) (end 132.207603 141.5) (width 0.2) (layer "F.Cu") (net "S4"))
 (segment (start 143.207603 141.5) (end 143.207603 142) (width 0.2) (layer "F.Cu") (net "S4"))
 (segment (start 143.207603 142) (end 143.207603 142.5) (width 0.2) (layer "F.Cu") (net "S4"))
 (segment (start 134.207603 142.5) (end 134.207603 142) (width 0.2) (layer "F.Cu") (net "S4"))
 (segment (start 133.207603 141.5) (end 133.207603 142) (width 0.2) (layer "F.Cu") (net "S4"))
 (segment (start 139.207603 142) (end 139.207603 142.5) (width 0.2) (layer "F.Cu") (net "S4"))
 (segment (start 130.207603 142) (end 130.207603 141.5) (width 0.2) (layer "F.Cu") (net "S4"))
 (segment (start 135.207603 141.5) (end 135.207603 142) (width 0.2) (layer "F.Cu") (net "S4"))
 (segment (start 133.207603 142) (end 133.207603 142.5) (width 0.2) (layer "F.Cu") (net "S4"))
 (segment (start 122 142) (end 128.707603 142) (width 0.2) (layer "F.Cu") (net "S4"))
 (segment (start 135.207603 142) (end 135.207603 142.5) (width 0.2) (layer "F.Cu") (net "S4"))
 (segment (start 130.207603 142.5) (end 130.207603 142) (width 0.2) (layer "F.Cu") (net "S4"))
 (segment (start 132.207603 142.5) (end 132.207603 142) (width 0.2) (layer "F.Cu") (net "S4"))
 (segment (start 147.207603 142) (end 147.207603 142.5) (width 0.2) (layer "F.Cu") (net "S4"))
 (segment (start 150.707603 142) (end 151.493707 142) (width 0.2) (layer "F.Cu") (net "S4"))
 (segment (start 145.207603 142) (end 145.207603 142.5) (width 0.2) (layer "F.Cu") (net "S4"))
 (segment (start 146.207603 142) (end 146.207603 141.5) (width 0.2) (layer "F.Cu") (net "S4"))
 (segment (start 145.207603 141.5) (end 145.207603 142) (width 0.2) (layer "F.Cu") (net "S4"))
 (segment (start 106 145) (end 118.585786 145) (width 0.2) (layer "F.Cu") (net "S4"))
 (segment (start 136.207603 142.5) (end 136.207603 142) (width 0.2) (layer "F.Cu") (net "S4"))
 (segment (start 139.207603 141.5) (end 139.207603 142) (width 0.2) (layer "F.Cu") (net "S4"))
 (segment (start 144.207603 142) (end 144.207603 141.5) (width 0.2) (layer "F.Cu") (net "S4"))
 (arc (start 128.707603 142) (mid 129.061156 142.146447) (end 129.207603 142.5) (width 0.2) (layer "F.Cu") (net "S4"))
 (arc (start 137.207603 142.5) (mid 137.35405 142.853553) (end 137.707603 143) (width 0.2) (layer "F.Cu") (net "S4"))
 (arc (start 134.207603 141.5) (mid 134.35405 141.146447) (end 134.707603 141) (width 0.2) (layer "F.Cu") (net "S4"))
 (arc (start 143.707603 143) (mid 144.061156 142.853553) (end 144.207603 142.5) (width 0.2) (layer "F.Cu") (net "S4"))
 (arc (start 118.585786 145) (mid 118.96847 144.92388) (end 119.292893 144.707107) (width 0.2) (layer "F.Cu") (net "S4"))
 (arc (start 136.707603 141) (mid 137.061156 141.146447) (end 137.207603 141.5) (width 0.2) (layer "F.Cu") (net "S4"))
 (arc (start 150.207603 142.5) (mid 150.35405 142.146447) (end 150.707603 142) (width 0.2) (layer "F.Cu") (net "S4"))
 (arc (start 140.207603 141.5) (mid 140.35405 141.146447) (end 140.707603 141) (width 0.2) (layer "F.Cu") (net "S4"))
 (arc (start 138.707603 141) (mid 139.061156 141.146447) (end 139.207603 141.5) (width 0.2) (layer "F.Cu") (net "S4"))
 (arc (start 136.207603 141.5) (mid 136.35405 141.146447) (end 136.707603 141) (width 0.2) (layer "F.Cu") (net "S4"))
 (arc (start 129.707603 143) (mid 130.061156 142.853553) (end 130.207603 142.5) (width 0.2) (layer "F.Cu") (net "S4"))
 (arc (start 131.707603 143) (mid 132.061156 142.853553) (end 132.207603 142.5) (width 0.2) (layer "F.Cu") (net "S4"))
 (arc (start 135.207603 142.5) (mid 135.35405 142.853553) (end 135.707603 143) (width 0.2) (layer "F.Cu") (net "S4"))
 (arc (start 149.707603 143) (mid 150.061156 142.853553) (end 150.207603 142.5) (width 0.2) (layer "F.Cu") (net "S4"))
 (arc (start 143.207603 142.5) (mid 143.35405 142.853553) (end 143.707603 143) (width 0.2) (layer "F.Cu") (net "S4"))
 (arc (start 131.207603 142.5) (mid 131.35405 142.853553) (end 131.707603 143) (width 0.2) (layer "F.Cu") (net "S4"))
 (arc (start 129.207603 142.5) (mid 129.35405 142.853553) (end 129.707603 143) (width 0.2) (layer "F.Cu") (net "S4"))
 (arc (start 141.207603 142.5) (mid 141.35405 142.853553) (end 141.707603 143) (width 0.2) (layer "F.Cu") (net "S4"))
 (arc (start 142.207603 141.5) (mid 142.35405 141.146447) (end 142.707603 141) (width 0.2) (layer "F.Cu") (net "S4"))
 (arc (start 132.707603 141) (mid 133.061156 141.146447) (end 133.207603 141.5) (width 0.2) (layer "F.Cu") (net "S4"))
 (arc (start 133.707603 143) (mid 134.061156 142.853553) (end 134.207603 142.5) (width 0.2) (layer "F.Cu") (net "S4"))
 (arc (start 147.707603 143) (mid 148.061156 142.853553) (end 148.207603 142.5) (width 0.2) (layer "F.Cu") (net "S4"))
 (arc (start 133.207603 142.5) (mid 133.35405 142.853553) (end 133.707603 143) (width 0.2) (layer "F.Cu") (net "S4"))
 (arc (start 130.207603 141.5) (mid 130.35405 141.146447) (end 130.707603 141) (width 0.2) (layer "F.Cu") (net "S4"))
 (arc (start 148.707603 141) (mid 149.061156 141.146447) (end 149.207603 141.5) (width 0.2) (layer "F.Cu") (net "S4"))
 (arc (start 138.207603 141.5) (mid 138.35405 141.146447) (end 138.707603 141) (width 0.2) (layer "F.Cu") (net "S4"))
 (arc (start 147.207603 142.5) (mid 147.35405 142.853553) (end 147.707603 143) (width 0.2) (layer "F.Cu") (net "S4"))
 (arc (start 135.707603 143) (mid 136.061156 142.853553) (end 136.207603 142.5) (width 0.2) (layer "F.Cu") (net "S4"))
 (arc (start 145.707603 143) (mid 146.061156 142.853553) (end 146.207603 142.5) (width 0.2) (layer "F.Cu") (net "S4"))
 (arc (start 144.707603 141) (mid 145.061156 141.146447) (end 145.207603 141.5) (width 0.2) (layer "F.Cu") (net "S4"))
 (arc (start 137.707603 143) (mid 138.061156 142.853553) (end 138.207603 142.5) (width 0.2) (layer "F.Cu") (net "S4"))
 (arc (start 146.207603 141.5) (mid 146.35405 141.146447) (end 146.707603 141) (width 0.2) (layer "F.Cu") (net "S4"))
 (arc (start 134.707603 141) (mid 135.061156 141.146447) (end 135.207603 141.5) (width 0.2) (layer "F.Cu") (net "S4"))
 (arc (start 142.707603 141) (mid 143.061156 141.146447) (end 143.207603 141.5) (width 0.2) (layer "F.Cu") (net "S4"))
 (arc (start 149.207603 142.5) (mid 149.35405 142.853553) (end 149.707603 143) (width 0.2) (layer "F.Cu") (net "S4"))
 (arc (start 130.707603 141) (mid 131.061156 141.146447) (end 131.207603 141.5) (width 0.2) (layer "F.Cu") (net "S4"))
 (arc (start 144.207603 141.5) (mid 144.35405 141.146447) (end 144.707603 141) (width 0.2) (layer "F.Cu") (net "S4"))
 (arc (start 139.207603 142.5) (mid 139.35405 142.853553) (end 139.707603 143) (width 0.2) (layer "F.Cu") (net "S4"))
 (arc (start 141.707603 143) (mid 142.061156 142.853553) (end 142.207603 142.5) (width 0.2) (layer "F.Cu") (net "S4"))
 (arc (start 132.207603 141.5) (mid 132.35405 141.146447) (end 132.707603 141) (width 0.2) (layer "F.Cu") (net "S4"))
 (arc (start 140.707603 141) (mid 141.061156 141.146447) (end 141.207603 141.5) (width 0.2) (layer "F.Cu") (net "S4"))
 (arc (start 139.707603 143) (mid 140.061156 142.853553) (end 140.207603 142.5) (width 0.2) (layer "F.Cu") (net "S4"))
 (arc (start 146.707603 141) (mid 147.061156 141.146447) (end 147.207603 141.5) (width 0.2) (layer "F.Cu") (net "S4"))
 (arc (start 148.207603 141.5) (mid 148.35405 141.146447) (end 148.707603 141) (width 0.2) (layer "F.Cu") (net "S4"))
 (arc (start 145.207603 142.5) (mid 145.35405 142.853553) (end 145.707603 143) (width 0.2) (layer "F.Cu") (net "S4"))
 (segment (start 124.292893 133.292893) (end 126.707107 135.707107) (width 0.25) (layer "F.Cu") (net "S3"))
 (segment (start 145.391988 132) (end 158.215131 132) (width 0.25) (layer "F.Cu") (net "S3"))
 (segment (start 158.215131 132) (end 164 132) (width 0.25) (layer "F.Cu") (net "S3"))
 (segment (start 142 132) (end 145.391988 132) (width 0.25) (layer "F.Cu") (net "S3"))
 (segment (start 138 136) (end 142 132) (width 0.25) (layer "F.Cu") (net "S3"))
 (segment (start 127.414214 136) (end 138 136) (width 0.25) (layer "F.Cu") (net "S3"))
 (segment (start 106 133) (end 123.585786 133) (width 0.25) (layer "F.Cu") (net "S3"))
 (arc (start 126.707107 135.707107) (mid 127.03153 135.92388) (end 127.414214 136) (width 0.25) (layer "F.Cu") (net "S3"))
 (arc (start 123.585786 133) (mid 123.96847 133.07612) (end 124.292893 133.292893) (width 0.25) (layer "F.Cu") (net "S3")))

